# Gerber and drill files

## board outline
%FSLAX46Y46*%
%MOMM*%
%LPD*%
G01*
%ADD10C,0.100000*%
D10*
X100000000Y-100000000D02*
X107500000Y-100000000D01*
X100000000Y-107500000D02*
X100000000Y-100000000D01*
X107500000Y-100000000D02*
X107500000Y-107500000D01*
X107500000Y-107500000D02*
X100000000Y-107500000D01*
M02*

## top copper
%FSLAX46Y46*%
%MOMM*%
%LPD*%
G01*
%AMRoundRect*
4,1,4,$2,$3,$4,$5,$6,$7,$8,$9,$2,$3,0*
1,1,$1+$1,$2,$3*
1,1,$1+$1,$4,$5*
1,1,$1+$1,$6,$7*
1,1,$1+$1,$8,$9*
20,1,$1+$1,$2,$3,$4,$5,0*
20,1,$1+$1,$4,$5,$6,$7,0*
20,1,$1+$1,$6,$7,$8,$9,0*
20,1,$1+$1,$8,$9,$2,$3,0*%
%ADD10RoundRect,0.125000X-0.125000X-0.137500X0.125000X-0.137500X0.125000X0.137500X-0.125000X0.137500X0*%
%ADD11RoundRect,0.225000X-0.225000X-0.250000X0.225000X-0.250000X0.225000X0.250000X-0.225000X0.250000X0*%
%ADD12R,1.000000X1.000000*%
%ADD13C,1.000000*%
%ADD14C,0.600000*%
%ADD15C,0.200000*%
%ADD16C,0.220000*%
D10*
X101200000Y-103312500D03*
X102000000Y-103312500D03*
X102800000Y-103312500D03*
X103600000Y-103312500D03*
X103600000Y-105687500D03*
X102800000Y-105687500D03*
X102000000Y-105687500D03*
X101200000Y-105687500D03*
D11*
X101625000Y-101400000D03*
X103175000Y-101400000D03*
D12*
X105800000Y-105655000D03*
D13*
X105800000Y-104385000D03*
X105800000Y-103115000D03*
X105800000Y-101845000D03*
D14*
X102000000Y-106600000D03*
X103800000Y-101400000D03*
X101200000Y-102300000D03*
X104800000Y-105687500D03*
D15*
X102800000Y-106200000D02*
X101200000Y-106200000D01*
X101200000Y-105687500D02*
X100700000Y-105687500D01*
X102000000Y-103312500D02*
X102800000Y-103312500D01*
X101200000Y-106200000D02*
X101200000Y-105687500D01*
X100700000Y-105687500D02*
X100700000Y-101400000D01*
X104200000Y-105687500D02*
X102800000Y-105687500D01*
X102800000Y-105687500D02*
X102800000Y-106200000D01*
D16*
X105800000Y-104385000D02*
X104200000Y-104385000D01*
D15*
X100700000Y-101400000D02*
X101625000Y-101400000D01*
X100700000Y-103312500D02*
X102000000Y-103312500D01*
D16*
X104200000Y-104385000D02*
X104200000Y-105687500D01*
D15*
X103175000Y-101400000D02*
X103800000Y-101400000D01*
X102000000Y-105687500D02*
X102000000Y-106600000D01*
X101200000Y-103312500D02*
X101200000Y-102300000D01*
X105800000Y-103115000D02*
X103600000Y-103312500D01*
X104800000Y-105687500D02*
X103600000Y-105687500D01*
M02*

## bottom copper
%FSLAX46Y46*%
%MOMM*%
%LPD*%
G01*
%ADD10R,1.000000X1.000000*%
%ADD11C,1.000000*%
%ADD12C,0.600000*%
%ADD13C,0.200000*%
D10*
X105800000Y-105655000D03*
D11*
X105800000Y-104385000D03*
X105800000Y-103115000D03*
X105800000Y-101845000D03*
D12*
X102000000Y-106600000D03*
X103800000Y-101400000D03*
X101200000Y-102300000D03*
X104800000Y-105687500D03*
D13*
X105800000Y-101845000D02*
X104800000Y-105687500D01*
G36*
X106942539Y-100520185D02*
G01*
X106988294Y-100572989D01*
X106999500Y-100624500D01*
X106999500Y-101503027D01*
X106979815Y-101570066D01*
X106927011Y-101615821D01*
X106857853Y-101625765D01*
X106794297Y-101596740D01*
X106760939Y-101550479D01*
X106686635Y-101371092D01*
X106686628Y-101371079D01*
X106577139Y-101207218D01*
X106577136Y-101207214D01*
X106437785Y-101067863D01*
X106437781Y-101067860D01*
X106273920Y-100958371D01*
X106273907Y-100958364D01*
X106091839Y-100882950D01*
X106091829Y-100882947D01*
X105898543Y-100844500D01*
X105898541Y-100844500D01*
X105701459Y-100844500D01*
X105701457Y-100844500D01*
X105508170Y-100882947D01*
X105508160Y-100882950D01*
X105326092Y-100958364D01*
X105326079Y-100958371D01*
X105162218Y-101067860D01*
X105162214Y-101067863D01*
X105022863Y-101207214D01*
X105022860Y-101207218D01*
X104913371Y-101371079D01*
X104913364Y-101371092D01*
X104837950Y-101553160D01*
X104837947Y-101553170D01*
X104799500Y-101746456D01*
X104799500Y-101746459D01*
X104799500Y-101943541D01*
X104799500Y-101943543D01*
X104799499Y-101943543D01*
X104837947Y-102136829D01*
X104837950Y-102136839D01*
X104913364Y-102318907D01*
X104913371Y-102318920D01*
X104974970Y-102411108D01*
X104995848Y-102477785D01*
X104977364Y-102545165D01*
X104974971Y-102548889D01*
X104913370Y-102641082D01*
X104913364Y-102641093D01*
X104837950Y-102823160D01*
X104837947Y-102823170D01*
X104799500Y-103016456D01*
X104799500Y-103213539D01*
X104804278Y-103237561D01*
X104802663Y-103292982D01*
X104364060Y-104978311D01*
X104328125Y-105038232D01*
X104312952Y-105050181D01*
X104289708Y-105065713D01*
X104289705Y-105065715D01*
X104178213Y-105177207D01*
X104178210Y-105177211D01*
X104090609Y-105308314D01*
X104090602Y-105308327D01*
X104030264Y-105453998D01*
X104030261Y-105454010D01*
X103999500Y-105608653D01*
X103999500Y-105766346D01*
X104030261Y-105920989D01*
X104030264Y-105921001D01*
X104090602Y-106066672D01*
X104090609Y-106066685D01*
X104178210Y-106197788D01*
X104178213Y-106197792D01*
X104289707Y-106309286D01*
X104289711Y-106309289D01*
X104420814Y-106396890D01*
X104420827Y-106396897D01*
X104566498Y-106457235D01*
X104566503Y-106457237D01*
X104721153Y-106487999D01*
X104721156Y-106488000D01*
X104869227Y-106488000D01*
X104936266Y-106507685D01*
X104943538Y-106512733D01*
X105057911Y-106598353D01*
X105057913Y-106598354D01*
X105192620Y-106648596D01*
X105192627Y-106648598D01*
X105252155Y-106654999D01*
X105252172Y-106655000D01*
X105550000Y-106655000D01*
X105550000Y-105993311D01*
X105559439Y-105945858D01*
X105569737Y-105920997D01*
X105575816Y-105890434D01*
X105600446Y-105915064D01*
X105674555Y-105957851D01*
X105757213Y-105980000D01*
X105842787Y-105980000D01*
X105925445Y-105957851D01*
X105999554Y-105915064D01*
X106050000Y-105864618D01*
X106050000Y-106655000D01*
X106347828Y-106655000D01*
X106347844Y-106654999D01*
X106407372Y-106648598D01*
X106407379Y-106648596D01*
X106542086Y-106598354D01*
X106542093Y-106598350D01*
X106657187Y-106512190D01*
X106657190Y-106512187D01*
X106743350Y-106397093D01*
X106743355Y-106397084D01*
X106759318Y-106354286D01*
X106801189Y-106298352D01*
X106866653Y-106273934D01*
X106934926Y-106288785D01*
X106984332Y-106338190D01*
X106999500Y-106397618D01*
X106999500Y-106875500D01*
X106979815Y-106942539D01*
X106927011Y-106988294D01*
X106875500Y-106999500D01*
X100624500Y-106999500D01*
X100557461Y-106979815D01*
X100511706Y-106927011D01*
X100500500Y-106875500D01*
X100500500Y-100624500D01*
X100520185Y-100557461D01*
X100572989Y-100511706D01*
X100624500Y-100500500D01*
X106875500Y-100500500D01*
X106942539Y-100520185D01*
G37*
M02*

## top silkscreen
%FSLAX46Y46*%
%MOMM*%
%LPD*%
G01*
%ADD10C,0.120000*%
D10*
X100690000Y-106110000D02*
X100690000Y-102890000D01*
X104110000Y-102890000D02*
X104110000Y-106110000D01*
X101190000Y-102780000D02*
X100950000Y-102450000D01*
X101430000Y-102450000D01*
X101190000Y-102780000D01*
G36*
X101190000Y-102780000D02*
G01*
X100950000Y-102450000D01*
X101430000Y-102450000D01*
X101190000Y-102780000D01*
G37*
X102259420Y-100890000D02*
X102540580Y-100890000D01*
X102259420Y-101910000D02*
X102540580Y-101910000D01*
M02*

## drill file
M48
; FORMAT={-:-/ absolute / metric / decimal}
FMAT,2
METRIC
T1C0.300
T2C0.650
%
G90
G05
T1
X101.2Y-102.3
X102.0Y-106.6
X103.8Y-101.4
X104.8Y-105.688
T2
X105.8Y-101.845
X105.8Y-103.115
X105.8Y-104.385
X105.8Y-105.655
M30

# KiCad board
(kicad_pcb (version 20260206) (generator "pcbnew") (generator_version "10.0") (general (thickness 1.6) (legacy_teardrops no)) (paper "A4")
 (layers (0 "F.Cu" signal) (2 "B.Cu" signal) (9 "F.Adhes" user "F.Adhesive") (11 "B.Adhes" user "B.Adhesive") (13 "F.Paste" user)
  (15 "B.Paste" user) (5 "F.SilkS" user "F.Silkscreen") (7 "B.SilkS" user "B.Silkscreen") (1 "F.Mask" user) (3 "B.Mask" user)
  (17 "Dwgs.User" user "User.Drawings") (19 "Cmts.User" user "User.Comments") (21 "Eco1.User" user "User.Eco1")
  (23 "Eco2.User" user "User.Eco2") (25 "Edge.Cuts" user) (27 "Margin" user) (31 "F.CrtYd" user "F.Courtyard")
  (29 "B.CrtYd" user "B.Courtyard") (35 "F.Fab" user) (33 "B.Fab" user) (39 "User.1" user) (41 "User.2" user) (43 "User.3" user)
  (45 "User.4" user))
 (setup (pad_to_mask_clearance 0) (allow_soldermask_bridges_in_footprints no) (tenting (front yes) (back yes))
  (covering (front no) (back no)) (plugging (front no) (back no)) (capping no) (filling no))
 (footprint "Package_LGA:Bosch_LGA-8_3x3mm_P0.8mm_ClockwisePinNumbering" (layer "F.Cu") (at 102.4 104.5)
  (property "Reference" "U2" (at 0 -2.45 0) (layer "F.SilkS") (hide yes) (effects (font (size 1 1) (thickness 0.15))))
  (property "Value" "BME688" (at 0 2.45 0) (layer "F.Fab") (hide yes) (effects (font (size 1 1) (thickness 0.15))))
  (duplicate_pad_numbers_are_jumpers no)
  (fp_line (start -1.71 1.61) (end -1.71 -1.61) (stroke (width 0.12) (type solid)) (layer "F.SilkS"))
  (fp_line (start 1.71 -1.61) (end 1.71 1.61) (stroke (width 0.12) (type solid)) (layer "F.SilkS"))
  (fp_poly (pts (xy -1.21 -1.72) (xy -1.45 -2.05) (xy -0.97 -2.05)) (stroke (width 0.12) (type solid)) (fill yes) (layer "F.SilkS"))
  (pad "1" smd roundrect (at -1.2 -1.1875) (size 0.5 0.525) (layers "F.Cu" "F.Mask" "F.Paste") (roundrect_rratio 0.25) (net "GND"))
  (pad "2" smd roundrect (at -0.4 -1.1875) (size 0.5 0.525) (layers "F.Cu" "F.Mask" "F.Paste") (roundrect_rratio 0.25) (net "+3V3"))
  (pad "3" smd roundrect (at 0.4 -1.1875) (size 0.5 0.525) (layers "F.Cu" "F.Mask" "F.Paste") (roundrect_rratio 0.25) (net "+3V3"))
  (pad "4" smd roundrect (at 1.2 -1.1875) (size 0.5 0.525) (layers "F.Cu" "F.Mask" "F.Paste") (roundrect_rratio 0.25) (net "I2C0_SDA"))
  (pad "5" smd roundrect (at 1.2 1.1875) (size 0.5 0.525) (layers "F.Cu" "F.Mask" "F.Paste") (roundrect_rratio 0.25) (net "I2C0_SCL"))
  (pad "6" smd roundrect (at 0.4 1.1875) (size 0.5 0.525) (layers "F.Cu" "F.Mask" "F.Paste") (roundrect_rratio 0.25) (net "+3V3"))
  (pad "7" smd roundrect (at -0.4 1.1875) (size 0.5 0.525) (layers "F.Cu" "F.Mask" "F.Paste") (roundrect_rratio 0.25) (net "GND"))
  (pad "8" smd roundrect (at -1.2 1.1875) (size 0.5 0.525) (layers "F.Cu" "F.Mask" "F.Paste") (roundrect_rratio 0.25) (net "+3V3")))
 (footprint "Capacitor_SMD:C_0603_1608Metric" (layer "F.Cu") (at 102.4 101.4)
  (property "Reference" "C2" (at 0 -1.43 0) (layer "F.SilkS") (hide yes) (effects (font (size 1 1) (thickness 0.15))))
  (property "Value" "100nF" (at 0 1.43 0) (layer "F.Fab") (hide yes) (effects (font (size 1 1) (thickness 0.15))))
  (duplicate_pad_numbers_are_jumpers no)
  (fp_line (start -0.14058 -0.51) (end 0.14058 -0.51) (stroke (width 0.12) (type solid)) (layer "F.SilkS"))
  (fp_line (start -0.14058 0.51) (end 0.14058 0.51) (stroke (width 0.12) (type solid)) (layer "F.SilkS"))
  (pad "1" smd roundrect (at -0.775 0) (size 0.9 0.95) (layers "F.Cu" "F.Mask" "F.Paste") (roundrect_rratio 0.25) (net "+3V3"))
  (pad "2" smd roundrect (at 0.775 0) (size 0.9 0.95) (layers "F.Cu" "F.Mask" "F.Paste") (roundrect_rratio 0.25) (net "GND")))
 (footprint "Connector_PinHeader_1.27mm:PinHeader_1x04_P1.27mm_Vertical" (layer "B.Cu") (at 105.8 105.655)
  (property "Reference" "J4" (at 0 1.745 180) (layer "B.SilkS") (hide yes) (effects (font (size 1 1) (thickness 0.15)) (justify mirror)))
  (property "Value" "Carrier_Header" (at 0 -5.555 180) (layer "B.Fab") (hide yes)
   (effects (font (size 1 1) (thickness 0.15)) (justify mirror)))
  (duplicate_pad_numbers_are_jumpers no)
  (pad "1" thru_hole rect (at 0 0) (size 1 1) (drill 0.65) (layers "*.Cu" "*.Mask") (remove_unused_layers no) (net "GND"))
  (pad "2" thru_hole circle (at 0 -1.27) (size 1 1) (drill 0.65) (layers "*.Cu" "*.Mask") (remove_unused_layers no) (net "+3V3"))
  (pad "3" thru_hole circle (at 0 -2.54) (size 1 1) (drill 0.65) (layers "*.Cu" "*.Mask") (remove_unused_layers no) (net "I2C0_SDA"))
  (pad "4" thru_hole circle (at 0 -3.81) (size 1 1) (drill 0.65) (layers "*.Cu" "*.Mask") (remove_unused_layers no) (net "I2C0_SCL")))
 (gr_line (start 100 100) (end 107.5 100) (stroke (width 0.1) (type default)) (layer "Edge.Cuts"))
 (gr_line (start 100 107.5) (end 100 100) (stroke (width 0.1) (type default)) (layer "Edge.Cuts"))
 (gr_line (start 107.5 100) (end 107.5 107.5) (stroke (width 0.1) (type default)) (layer "Edge.Cuts"))
 (gr_line (start 107.5 107.5) (end 100 107.5) (stroke (width 0.1) (type default)) (layer "Edge.Cuts"))
 (segment (start 102.8 106.2) (end 101.2 106.2) (width 0.2) (layer "F.Cu") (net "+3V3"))
 (segment (start 101.2 105.6875) (end 100.7 105.6875) (width 0.2) (layer "F.Cu") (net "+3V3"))
 (segment (start 102 103.3125) (end 102.8 103.3125) (width 0.2) (layer "F.Cu") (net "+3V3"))
 (segment (start 101.2 106.2) (end 101.2 105.6875) (width 0.2) (layer "F.Cu") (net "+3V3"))
 (segment (start 100.7 105.6875) (end 100.7 101.4) (width 0.2) (layer "F.Cu") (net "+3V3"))
 (segment (start 104.2 105.6875) (end 102.8 105.6875) (width 0.2) (layer "F.Cu") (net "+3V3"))
 (segment (start 102.8 105.6875) (end 102.8 106.2) (width 0.2) (layer "F.Cu") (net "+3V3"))
 (segment (start 105.8 104.385) (end 104.2 104.385) (width 0.22) (layer "F.Cu") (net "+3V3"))
 (segment (start 100.7 101.4) (end 101.625 101.4) (width 0.2) (layer "F.Cu") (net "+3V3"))
 (segment (start 100.7 103.3125) (end 102 103.3125) (width 0.2) (layer "F.Cu") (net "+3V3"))
 (segment (start 104.2 104.385) (end 104.2 105.6875) (width 0.22) (layer "F.Cu") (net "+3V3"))
 (segment (start 103.175 101.4) (end 103.8 101.4) (width 0.2) (layer "F.Cu") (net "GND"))
 (segment (start 102 105.6875) (end 102 106.6) (width 0.2) (layer "F.Cu") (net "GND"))
 (segment (start 101.2 103.3125) (end 101.2 102.3) (width 0.2) (layer "F.Cu") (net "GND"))
 (via (at 102 106.6) (size 0.6) (drill 0.3) (layers "F.Cu" "B.Cu") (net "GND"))
 (via (at 103.8 101.4) (size 0.6) (drill 0.3) (layers "F.Cu" "B.Cu") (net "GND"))
 (via (at 101.2 102.3) (size 0.6) (drill 0.3) (layers "F.Cu" "B.Cu") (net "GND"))
 (segment (start 105.8 103.115) (end 103.6 103.3125) (width 0.2) (layer "F.Cu") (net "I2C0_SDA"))
 (segment (start 104.8 105.6875) (end 103.6 105.6875) (width 0.2) (layer "F.Cu") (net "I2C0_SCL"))
 (via (at 104.8 105.6875) (size 0.6) (drill 0.3) (layers "F.Cu" "B.Cu") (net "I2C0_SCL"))
 (segment (start 105.8 101.845) (end 104.8 105.6875) (width 0.2) (layer "B.Cu") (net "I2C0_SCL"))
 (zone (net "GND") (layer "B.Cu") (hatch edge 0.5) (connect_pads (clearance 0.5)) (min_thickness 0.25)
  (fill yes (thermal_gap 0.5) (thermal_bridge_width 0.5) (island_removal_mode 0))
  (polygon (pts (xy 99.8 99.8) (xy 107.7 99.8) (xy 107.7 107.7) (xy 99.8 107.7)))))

